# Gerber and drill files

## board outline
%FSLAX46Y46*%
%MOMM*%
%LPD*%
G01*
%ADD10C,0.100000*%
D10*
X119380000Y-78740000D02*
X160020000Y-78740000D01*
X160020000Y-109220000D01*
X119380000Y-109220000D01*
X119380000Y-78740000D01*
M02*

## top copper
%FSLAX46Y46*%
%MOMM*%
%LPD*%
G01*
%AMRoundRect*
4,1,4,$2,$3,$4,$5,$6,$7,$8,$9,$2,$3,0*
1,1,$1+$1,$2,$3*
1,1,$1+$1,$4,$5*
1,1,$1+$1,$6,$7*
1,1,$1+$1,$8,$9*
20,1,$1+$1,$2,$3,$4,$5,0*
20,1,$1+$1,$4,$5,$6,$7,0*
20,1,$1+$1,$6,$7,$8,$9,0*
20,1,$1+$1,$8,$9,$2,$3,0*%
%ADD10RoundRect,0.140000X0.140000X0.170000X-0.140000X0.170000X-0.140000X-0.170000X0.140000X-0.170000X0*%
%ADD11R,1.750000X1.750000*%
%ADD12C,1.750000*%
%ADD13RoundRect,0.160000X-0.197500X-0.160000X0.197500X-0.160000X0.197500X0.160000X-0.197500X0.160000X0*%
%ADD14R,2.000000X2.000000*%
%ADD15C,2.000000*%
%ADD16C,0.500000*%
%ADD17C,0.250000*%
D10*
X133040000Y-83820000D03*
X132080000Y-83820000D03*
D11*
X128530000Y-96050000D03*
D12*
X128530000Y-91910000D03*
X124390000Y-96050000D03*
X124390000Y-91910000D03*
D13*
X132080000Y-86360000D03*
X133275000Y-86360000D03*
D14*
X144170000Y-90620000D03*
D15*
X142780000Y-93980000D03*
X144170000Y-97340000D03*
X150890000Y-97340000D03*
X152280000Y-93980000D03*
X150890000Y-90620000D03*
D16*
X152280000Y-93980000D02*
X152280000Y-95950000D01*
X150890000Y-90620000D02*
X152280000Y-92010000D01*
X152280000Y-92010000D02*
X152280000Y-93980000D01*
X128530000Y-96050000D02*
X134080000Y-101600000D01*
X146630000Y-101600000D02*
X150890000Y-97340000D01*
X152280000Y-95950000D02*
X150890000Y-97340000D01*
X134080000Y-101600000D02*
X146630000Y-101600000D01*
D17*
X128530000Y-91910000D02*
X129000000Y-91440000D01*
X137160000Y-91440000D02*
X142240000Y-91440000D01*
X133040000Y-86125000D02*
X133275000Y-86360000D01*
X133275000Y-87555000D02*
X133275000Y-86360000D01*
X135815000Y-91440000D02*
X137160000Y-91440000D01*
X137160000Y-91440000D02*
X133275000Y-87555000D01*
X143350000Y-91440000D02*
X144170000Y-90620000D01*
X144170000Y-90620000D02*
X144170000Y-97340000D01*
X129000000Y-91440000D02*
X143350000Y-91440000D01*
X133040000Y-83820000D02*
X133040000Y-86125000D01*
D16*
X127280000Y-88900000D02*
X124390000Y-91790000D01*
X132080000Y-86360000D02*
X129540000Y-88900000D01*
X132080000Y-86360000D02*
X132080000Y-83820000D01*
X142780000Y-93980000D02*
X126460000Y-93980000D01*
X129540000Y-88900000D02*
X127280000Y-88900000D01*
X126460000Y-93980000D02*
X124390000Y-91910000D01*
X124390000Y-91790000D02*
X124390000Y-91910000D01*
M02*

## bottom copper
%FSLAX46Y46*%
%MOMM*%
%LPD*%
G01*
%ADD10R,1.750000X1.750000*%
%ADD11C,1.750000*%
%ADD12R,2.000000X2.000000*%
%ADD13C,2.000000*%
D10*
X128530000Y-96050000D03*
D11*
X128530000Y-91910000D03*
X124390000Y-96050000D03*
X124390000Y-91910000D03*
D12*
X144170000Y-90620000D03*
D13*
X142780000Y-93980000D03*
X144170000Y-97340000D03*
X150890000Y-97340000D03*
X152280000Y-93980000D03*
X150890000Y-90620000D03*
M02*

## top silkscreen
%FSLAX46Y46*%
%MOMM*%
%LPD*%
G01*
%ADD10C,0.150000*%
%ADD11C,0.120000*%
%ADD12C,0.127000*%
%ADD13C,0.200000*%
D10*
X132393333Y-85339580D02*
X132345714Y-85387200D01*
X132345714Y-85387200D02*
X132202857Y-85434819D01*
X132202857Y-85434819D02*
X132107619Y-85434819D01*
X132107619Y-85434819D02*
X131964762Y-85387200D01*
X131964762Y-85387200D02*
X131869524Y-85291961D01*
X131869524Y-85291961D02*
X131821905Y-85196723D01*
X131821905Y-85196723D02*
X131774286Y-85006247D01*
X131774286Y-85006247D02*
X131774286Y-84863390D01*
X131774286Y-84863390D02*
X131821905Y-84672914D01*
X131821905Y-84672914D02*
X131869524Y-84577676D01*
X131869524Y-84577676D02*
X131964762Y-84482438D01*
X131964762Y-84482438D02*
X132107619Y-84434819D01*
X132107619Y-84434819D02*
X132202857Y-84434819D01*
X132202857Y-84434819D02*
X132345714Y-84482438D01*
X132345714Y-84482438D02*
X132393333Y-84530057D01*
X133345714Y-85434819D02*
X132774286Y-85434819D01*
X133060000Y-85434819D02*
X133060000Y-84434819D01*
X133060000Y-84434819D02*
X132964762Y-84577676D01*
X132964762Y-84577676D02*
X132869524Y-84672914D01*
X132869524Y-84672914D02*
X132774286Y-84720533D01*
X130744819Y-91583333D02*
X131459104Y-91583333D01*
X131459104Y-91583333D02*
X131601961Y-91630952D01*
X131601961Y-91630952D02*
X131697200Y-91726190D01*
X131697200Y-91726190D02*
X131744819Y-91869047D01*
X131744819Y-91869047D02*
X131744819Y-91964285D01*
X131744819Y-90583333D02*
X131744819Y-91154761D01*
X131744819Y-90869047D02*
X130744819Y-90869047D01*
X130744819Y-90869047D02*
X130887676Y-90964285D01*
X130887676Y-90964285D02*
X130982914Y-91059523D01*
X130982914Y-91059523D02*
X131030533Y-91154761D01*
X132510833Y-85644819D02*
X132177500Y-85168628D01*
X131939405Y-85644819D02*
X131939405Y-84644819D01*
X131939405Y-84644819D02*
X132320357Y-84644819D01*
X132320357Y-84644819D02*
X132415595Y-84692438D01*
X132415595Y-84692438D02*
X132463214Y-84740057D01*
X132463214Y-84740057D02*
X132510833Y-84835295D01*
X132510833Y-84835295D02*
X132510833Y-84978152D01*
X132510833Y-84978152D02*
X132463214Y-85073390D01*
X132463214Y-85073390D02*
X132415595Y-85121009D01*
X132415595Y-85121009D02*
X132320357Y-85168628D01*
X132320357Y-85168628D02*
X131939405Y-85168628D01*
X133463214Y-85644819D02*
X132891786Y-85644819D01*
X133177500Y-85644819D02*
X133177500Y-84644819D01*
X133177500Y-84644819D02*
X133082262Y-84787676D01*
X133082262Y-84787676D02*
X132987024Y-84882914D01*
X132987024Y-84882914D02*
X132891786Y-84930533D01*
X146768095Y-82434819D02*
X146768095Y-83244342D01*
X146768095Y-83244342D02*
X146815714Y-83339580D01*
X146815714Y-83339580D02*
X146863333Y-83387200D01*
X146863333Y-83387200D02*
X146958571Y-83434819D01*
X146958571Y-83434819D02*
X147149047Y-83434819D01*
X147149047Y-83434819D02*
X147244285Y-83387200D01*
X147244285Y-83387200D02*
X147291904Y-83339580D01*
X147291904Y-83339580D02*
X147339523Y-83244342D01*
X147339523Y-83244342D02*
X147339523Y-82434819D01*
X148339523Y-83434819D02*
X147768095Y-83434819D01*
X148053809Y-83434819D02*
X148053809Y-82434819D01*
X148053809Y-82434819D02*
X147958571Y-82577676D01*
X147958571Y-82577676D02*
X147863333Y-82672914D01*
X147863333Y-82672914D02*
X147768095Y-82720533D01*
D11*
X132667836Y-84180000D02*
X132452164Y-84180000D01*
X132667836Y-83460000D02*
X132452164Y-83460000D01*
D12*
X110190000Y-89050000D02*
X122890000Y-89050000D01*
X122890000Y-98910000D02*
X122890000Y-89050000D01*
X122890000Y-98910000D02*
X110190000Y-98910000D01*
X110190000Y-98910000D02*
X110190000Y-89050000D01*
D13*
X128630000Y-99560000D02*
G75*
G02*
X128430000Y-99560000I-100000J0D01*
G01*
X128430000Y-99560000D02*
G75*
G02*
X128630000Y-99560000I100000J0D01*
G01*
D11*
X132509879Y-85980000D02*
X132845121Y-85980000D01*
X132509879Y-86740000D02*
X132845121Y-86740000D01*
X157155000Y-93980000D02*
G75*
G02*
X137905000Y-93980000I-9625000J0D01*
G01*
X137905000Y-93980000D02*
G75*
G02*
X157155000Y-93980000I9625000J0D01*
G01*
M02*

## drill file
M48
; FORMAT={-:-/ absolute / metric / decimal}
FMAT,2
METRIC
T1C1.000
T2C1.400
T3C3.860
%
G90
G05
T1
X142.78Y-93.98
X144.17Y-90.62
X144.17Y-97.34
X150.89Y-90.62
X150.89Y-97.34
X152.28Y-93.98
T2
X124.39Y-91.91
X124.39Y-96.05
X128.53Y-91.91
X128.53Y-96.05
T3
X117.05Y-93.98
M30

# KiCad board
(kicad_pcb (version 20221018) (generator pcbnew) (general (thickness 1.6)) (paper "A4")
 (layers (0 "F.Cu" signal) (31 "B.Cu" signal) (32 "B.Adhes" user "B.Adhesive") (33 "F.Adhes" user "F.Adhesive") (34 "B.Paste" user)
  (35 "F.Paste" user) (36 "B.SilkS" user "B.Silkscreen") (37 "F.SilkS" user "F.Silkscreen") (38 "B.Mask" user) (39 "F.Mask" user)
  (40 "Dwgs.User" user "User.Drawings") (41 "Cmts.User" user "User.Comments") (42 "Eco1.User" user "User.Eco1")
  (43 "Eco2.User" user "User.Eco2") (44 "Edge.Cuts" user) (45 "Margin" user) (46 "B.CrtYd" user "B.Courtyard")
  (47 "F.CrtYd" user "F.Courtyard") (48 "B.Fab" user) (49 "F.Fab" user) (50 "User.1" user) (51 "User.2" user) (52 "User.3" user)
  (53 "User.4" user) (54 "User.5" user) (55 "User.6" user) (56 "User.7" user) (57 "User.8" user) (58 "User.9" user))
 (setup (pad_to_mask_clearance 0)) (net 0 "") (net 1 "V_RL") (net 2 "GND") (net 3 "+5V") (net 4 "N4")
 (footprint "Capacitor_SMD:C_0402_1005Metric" (layer "F.Cu") (at 132.56 83.82 180)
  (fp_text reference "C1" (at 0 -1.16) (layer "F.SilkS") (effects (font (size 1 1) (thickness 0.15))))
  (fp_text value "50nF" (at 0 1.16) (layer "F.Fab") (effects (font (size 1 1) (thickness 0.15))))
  (fp_line (start -0.107836 -0.36) (end 0.107836 -0.36) (stroke (width 0.12) (type solid)) (layer "F.SilkS"))
  (fp_line (start -0.107836 0.36) (end 0.107836 0.36) (stroke (width 0.12) (type solid)) (layer "F.SilkS"))
  (pad "1" smd roundrect (at -0.48 0 180) (size 0.56 0.62) (layers "F.Cu" "F.Paste" "F.Mask") (roundrect_rratio 0.25) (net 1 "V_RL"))
  (pad "2" smd roundrect (at 0.48 0 180) (size 0.56 0.62) (layers "F.Cu" "F.Paste" "F.Mask") (roundrect_rratio 0.25) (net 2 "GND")))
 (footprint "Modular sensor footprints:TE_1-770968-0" (layer "F.Cu") (at 128.53 96.05 -90)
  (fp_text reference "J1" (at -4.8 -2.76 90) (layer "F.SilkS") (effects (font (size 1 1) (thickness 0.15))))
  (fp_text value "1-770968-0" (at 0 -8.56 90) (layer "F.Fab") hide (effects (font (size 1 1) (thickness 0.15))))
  (fp_line (start -7 18.34) (end -7 5.64) (stroke (width 0.127) (type solid)) (layer "F.SilkS"))
  (fp_line (start 2.86 5.64) (end -7 5.64) (stroke (width 0.127) (type solid)) (layer "F.SilkS"))
  (fp_line (start 2.86 5.64) (end 2.86 18.34) (stroke (width 0.127) (type solid)) (layer "F.SilkS"))
  (fp_line (start 2.86 18.34) (end -7 18.34) (stroke (width 0.127) (type solid)) (layer "F.SilkS"))
  (fp_circle (center 3.51 0) (end 3.61 0) (stroke (width 0.2) (type solid)) (fill none) (layer "F.SilkS"))
  (pad "" np_thru_hole circle (at -2.07 11.48 270) (size 3.86 3.86) (drill 3.86) (layers "*.Cu" "*.Mask"))
  (pad "1" thru_hole rect (at 0 0 270) (size 1.75 1.75) (drill 1.4) (layers "*.Cu" "*.Mask") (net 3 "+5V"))
  (pad "2" thru_hole circle (at -4.14 0 270) (size 1.75 1.75) (drill 1.4) (layers "*.Cu" "*.Mask") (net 1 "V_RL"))
  (pad "3" thru_hole circle (at 0 4.14 270) (size 1.75 1.75) (drill 1.4) (layers "*.Cu" "*.Mask") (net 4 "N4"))
  (pad "4" thru_hole circle (at -4.14 4.14 270) (size 1.75 1.75) (drill 1.4) (layers "*.Cu" "*.Mask") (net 2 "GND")))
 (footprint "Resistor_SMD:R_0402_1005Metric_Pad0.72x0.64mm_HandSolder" (layer "F.Cu") (at 132.6775 86.36)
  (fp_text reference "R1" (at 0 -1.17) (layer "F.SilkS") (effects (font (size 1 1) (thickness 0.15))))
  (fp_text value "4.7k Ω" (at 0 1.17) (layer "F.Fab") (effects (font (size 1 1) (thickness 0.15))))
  (fp_line (start -0.167621 -0.38) (end 0.167621 -0.38) (stroke (width 0.12) (type solid)) (layer "F.SilkS"))
  (fp_line (start -0.167621 0.38) (end 0.167621 0.38) (stroke (width 0.12) (type solid)) (layer "F.SilkS"))
  (pad "1" smd roundrect (at -0.5975 0) (size 0.715 0.64) (layers "F.Cu" "F.Paste" "F.Mask") (roundrect_rratio 0.25) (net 2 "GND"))
  (pad "2" smd roundrect (at 0.5975 0) (size 0.715 0.64) (layers "F.Cu" "F.Paste" "F.Mask") (roundrect_rratio 0.25) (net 1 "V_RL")))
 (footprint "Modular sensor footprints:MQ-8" (layer "F.Cu") (at 144.17 90.62)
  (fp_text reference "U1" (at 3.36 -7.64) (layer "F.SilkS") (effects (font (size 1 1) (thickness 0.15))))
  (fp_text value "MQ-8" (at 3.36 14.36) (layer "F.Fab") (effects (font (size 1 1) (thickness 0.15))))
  (fp_circle (center 3.36 3.36) (end 12.985 3.36) (stroke (width 0.12) (type solid)) (fill none) (layer "F.SilkS"))
  (pad "1" thru_hole rect (at 0 0) (size 2 2) (drill 1) (layers "*.Cu" "*.Mask") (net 1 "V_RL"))
  (pad "2" thru_hole circle (at -1.39 3.36) (size 2 2) (drill 1) (layers "*.Cu" "*.Mask") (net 2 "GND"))
  (pad "3" thru_hole circle (at 0 6.72 90) (size 2 2) (drill 1) (layers "*.Cu" "*.Mask") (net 1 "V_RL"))
  (pad "4" thru_hole circle (at 6.72 6.72 180) (size 2 2) (drill 1) (layers "*.Cu" "*.Mask") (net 3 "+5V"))
  (pad "5" thru_hole circle (at 8.11 3.36) (size 2 2) (drill 1) (layers "*.Cu" "*.Mask") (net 3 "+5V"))
  (pad "6" thru_hole circle (at 6.72 0 270) (size 2 2) (drill 1) (layers "*.Cu" "*.Mask") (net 3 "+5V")))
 (gr_rect (start 119.38 78.74) (end 160.02 109.22) (stroke (width 0.1) (type default)) (fill none) (layer "Edge.Cuts"))
 (segment (start 152.28 93.98) (end 152.28 95.95) (width 0.5) (layer "F.Cu") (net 3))
 (segment (start 150.89 90.62) (end 152.28 92.01) (width 0.5) (layer "F.Cu") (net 3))
 (segment (start 152.28 92.01) (end 152.28 93.98) (width 0.5) (layer "F.Cu") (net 3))
 (segment (start 128.53 96.05) (end 134.08 101.6) (width 0.5) (layer "F.Cu") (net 3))
 (segment (start 146.63 101.6) (end 150.89 97.34) (width 0.5) (layer "F.Cu") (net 3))
 (segment (start 152.28 95.95) (end 150.89 97.34) (width 0.5) (layer "F.Cu") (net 3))
 (segment (start 134.08 101.6) (end 146.63 101.6) (width 0.5) (layer "F.Cu") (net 3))
 (segment (start 128.53 91.91) (end 129 91.44) (width 0.25) (layer "F.Cu") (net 1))
 (segment (start 137.16 91.44) (end 142.24 91.44) (width 0.25) (layer "F.Cu") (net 1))
 (segment (start 133.04 86.125) (end 133.275 86.36) (width 0.25) (layer "F.Cu") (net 1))
 (segment (start 133.275 87.555) (end 133.275 86.36) (width 0.25) (layer "F.Cu") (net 1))
 (segment (start 135.815 91.44) (end 137.16 91.44) (width 0.25) (layer "F.Cu") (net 1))
 (segment (start 137.16 91.44) (end 133.275 87.555) (width 0.25) (layer "F.Cu") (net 1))
 (segment (start 143.35 91.44) (end 144.17 90.62) (width 0.25) (layer "F.Cu") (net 1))
 (segment (start 144.17 90.62) (end 144.17 97.34) (width 0.25) (layer "F.Cu") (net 1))
 (segment (start 129 91.44) (end 143.35 91.44) (width 0.25) (layer "F.Cu") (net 1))
 (segment (start 133.04 83.82) (end 133.04 86.125) (width 0.25) (layer "F.Cu") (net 1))
 (segment (start 127.28 88.9) (end 124.39 91.79) (width 0.5) (layer "F.Cu") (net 2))
 (segment (start 132.08 86.36) (end 129.54 88.9) (width 0.5) (layer "F.Cu") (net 2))
 (segment (start 132.08 86.36) (end 132.08 83.82) (width 0.5) (layer "F.Cu") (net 2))
 (segment (start 142.78 93.98) (end 126.46 93.98) (width 0.5) (layer "F.Cu") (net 2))
 (segment (start 129.54 88.9) (end 127.28 88.9) (width 0.5) (layer "F.Cu") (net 2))
 (segment (start 126.46 93.98) (end 124.39 91.91) (width 0.5) (layer "F.Cu") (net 2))
 (segment (start 124.39 91.79) (end 124.39 91.91) (width 0.5) (layer "F.Cu") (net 2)))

